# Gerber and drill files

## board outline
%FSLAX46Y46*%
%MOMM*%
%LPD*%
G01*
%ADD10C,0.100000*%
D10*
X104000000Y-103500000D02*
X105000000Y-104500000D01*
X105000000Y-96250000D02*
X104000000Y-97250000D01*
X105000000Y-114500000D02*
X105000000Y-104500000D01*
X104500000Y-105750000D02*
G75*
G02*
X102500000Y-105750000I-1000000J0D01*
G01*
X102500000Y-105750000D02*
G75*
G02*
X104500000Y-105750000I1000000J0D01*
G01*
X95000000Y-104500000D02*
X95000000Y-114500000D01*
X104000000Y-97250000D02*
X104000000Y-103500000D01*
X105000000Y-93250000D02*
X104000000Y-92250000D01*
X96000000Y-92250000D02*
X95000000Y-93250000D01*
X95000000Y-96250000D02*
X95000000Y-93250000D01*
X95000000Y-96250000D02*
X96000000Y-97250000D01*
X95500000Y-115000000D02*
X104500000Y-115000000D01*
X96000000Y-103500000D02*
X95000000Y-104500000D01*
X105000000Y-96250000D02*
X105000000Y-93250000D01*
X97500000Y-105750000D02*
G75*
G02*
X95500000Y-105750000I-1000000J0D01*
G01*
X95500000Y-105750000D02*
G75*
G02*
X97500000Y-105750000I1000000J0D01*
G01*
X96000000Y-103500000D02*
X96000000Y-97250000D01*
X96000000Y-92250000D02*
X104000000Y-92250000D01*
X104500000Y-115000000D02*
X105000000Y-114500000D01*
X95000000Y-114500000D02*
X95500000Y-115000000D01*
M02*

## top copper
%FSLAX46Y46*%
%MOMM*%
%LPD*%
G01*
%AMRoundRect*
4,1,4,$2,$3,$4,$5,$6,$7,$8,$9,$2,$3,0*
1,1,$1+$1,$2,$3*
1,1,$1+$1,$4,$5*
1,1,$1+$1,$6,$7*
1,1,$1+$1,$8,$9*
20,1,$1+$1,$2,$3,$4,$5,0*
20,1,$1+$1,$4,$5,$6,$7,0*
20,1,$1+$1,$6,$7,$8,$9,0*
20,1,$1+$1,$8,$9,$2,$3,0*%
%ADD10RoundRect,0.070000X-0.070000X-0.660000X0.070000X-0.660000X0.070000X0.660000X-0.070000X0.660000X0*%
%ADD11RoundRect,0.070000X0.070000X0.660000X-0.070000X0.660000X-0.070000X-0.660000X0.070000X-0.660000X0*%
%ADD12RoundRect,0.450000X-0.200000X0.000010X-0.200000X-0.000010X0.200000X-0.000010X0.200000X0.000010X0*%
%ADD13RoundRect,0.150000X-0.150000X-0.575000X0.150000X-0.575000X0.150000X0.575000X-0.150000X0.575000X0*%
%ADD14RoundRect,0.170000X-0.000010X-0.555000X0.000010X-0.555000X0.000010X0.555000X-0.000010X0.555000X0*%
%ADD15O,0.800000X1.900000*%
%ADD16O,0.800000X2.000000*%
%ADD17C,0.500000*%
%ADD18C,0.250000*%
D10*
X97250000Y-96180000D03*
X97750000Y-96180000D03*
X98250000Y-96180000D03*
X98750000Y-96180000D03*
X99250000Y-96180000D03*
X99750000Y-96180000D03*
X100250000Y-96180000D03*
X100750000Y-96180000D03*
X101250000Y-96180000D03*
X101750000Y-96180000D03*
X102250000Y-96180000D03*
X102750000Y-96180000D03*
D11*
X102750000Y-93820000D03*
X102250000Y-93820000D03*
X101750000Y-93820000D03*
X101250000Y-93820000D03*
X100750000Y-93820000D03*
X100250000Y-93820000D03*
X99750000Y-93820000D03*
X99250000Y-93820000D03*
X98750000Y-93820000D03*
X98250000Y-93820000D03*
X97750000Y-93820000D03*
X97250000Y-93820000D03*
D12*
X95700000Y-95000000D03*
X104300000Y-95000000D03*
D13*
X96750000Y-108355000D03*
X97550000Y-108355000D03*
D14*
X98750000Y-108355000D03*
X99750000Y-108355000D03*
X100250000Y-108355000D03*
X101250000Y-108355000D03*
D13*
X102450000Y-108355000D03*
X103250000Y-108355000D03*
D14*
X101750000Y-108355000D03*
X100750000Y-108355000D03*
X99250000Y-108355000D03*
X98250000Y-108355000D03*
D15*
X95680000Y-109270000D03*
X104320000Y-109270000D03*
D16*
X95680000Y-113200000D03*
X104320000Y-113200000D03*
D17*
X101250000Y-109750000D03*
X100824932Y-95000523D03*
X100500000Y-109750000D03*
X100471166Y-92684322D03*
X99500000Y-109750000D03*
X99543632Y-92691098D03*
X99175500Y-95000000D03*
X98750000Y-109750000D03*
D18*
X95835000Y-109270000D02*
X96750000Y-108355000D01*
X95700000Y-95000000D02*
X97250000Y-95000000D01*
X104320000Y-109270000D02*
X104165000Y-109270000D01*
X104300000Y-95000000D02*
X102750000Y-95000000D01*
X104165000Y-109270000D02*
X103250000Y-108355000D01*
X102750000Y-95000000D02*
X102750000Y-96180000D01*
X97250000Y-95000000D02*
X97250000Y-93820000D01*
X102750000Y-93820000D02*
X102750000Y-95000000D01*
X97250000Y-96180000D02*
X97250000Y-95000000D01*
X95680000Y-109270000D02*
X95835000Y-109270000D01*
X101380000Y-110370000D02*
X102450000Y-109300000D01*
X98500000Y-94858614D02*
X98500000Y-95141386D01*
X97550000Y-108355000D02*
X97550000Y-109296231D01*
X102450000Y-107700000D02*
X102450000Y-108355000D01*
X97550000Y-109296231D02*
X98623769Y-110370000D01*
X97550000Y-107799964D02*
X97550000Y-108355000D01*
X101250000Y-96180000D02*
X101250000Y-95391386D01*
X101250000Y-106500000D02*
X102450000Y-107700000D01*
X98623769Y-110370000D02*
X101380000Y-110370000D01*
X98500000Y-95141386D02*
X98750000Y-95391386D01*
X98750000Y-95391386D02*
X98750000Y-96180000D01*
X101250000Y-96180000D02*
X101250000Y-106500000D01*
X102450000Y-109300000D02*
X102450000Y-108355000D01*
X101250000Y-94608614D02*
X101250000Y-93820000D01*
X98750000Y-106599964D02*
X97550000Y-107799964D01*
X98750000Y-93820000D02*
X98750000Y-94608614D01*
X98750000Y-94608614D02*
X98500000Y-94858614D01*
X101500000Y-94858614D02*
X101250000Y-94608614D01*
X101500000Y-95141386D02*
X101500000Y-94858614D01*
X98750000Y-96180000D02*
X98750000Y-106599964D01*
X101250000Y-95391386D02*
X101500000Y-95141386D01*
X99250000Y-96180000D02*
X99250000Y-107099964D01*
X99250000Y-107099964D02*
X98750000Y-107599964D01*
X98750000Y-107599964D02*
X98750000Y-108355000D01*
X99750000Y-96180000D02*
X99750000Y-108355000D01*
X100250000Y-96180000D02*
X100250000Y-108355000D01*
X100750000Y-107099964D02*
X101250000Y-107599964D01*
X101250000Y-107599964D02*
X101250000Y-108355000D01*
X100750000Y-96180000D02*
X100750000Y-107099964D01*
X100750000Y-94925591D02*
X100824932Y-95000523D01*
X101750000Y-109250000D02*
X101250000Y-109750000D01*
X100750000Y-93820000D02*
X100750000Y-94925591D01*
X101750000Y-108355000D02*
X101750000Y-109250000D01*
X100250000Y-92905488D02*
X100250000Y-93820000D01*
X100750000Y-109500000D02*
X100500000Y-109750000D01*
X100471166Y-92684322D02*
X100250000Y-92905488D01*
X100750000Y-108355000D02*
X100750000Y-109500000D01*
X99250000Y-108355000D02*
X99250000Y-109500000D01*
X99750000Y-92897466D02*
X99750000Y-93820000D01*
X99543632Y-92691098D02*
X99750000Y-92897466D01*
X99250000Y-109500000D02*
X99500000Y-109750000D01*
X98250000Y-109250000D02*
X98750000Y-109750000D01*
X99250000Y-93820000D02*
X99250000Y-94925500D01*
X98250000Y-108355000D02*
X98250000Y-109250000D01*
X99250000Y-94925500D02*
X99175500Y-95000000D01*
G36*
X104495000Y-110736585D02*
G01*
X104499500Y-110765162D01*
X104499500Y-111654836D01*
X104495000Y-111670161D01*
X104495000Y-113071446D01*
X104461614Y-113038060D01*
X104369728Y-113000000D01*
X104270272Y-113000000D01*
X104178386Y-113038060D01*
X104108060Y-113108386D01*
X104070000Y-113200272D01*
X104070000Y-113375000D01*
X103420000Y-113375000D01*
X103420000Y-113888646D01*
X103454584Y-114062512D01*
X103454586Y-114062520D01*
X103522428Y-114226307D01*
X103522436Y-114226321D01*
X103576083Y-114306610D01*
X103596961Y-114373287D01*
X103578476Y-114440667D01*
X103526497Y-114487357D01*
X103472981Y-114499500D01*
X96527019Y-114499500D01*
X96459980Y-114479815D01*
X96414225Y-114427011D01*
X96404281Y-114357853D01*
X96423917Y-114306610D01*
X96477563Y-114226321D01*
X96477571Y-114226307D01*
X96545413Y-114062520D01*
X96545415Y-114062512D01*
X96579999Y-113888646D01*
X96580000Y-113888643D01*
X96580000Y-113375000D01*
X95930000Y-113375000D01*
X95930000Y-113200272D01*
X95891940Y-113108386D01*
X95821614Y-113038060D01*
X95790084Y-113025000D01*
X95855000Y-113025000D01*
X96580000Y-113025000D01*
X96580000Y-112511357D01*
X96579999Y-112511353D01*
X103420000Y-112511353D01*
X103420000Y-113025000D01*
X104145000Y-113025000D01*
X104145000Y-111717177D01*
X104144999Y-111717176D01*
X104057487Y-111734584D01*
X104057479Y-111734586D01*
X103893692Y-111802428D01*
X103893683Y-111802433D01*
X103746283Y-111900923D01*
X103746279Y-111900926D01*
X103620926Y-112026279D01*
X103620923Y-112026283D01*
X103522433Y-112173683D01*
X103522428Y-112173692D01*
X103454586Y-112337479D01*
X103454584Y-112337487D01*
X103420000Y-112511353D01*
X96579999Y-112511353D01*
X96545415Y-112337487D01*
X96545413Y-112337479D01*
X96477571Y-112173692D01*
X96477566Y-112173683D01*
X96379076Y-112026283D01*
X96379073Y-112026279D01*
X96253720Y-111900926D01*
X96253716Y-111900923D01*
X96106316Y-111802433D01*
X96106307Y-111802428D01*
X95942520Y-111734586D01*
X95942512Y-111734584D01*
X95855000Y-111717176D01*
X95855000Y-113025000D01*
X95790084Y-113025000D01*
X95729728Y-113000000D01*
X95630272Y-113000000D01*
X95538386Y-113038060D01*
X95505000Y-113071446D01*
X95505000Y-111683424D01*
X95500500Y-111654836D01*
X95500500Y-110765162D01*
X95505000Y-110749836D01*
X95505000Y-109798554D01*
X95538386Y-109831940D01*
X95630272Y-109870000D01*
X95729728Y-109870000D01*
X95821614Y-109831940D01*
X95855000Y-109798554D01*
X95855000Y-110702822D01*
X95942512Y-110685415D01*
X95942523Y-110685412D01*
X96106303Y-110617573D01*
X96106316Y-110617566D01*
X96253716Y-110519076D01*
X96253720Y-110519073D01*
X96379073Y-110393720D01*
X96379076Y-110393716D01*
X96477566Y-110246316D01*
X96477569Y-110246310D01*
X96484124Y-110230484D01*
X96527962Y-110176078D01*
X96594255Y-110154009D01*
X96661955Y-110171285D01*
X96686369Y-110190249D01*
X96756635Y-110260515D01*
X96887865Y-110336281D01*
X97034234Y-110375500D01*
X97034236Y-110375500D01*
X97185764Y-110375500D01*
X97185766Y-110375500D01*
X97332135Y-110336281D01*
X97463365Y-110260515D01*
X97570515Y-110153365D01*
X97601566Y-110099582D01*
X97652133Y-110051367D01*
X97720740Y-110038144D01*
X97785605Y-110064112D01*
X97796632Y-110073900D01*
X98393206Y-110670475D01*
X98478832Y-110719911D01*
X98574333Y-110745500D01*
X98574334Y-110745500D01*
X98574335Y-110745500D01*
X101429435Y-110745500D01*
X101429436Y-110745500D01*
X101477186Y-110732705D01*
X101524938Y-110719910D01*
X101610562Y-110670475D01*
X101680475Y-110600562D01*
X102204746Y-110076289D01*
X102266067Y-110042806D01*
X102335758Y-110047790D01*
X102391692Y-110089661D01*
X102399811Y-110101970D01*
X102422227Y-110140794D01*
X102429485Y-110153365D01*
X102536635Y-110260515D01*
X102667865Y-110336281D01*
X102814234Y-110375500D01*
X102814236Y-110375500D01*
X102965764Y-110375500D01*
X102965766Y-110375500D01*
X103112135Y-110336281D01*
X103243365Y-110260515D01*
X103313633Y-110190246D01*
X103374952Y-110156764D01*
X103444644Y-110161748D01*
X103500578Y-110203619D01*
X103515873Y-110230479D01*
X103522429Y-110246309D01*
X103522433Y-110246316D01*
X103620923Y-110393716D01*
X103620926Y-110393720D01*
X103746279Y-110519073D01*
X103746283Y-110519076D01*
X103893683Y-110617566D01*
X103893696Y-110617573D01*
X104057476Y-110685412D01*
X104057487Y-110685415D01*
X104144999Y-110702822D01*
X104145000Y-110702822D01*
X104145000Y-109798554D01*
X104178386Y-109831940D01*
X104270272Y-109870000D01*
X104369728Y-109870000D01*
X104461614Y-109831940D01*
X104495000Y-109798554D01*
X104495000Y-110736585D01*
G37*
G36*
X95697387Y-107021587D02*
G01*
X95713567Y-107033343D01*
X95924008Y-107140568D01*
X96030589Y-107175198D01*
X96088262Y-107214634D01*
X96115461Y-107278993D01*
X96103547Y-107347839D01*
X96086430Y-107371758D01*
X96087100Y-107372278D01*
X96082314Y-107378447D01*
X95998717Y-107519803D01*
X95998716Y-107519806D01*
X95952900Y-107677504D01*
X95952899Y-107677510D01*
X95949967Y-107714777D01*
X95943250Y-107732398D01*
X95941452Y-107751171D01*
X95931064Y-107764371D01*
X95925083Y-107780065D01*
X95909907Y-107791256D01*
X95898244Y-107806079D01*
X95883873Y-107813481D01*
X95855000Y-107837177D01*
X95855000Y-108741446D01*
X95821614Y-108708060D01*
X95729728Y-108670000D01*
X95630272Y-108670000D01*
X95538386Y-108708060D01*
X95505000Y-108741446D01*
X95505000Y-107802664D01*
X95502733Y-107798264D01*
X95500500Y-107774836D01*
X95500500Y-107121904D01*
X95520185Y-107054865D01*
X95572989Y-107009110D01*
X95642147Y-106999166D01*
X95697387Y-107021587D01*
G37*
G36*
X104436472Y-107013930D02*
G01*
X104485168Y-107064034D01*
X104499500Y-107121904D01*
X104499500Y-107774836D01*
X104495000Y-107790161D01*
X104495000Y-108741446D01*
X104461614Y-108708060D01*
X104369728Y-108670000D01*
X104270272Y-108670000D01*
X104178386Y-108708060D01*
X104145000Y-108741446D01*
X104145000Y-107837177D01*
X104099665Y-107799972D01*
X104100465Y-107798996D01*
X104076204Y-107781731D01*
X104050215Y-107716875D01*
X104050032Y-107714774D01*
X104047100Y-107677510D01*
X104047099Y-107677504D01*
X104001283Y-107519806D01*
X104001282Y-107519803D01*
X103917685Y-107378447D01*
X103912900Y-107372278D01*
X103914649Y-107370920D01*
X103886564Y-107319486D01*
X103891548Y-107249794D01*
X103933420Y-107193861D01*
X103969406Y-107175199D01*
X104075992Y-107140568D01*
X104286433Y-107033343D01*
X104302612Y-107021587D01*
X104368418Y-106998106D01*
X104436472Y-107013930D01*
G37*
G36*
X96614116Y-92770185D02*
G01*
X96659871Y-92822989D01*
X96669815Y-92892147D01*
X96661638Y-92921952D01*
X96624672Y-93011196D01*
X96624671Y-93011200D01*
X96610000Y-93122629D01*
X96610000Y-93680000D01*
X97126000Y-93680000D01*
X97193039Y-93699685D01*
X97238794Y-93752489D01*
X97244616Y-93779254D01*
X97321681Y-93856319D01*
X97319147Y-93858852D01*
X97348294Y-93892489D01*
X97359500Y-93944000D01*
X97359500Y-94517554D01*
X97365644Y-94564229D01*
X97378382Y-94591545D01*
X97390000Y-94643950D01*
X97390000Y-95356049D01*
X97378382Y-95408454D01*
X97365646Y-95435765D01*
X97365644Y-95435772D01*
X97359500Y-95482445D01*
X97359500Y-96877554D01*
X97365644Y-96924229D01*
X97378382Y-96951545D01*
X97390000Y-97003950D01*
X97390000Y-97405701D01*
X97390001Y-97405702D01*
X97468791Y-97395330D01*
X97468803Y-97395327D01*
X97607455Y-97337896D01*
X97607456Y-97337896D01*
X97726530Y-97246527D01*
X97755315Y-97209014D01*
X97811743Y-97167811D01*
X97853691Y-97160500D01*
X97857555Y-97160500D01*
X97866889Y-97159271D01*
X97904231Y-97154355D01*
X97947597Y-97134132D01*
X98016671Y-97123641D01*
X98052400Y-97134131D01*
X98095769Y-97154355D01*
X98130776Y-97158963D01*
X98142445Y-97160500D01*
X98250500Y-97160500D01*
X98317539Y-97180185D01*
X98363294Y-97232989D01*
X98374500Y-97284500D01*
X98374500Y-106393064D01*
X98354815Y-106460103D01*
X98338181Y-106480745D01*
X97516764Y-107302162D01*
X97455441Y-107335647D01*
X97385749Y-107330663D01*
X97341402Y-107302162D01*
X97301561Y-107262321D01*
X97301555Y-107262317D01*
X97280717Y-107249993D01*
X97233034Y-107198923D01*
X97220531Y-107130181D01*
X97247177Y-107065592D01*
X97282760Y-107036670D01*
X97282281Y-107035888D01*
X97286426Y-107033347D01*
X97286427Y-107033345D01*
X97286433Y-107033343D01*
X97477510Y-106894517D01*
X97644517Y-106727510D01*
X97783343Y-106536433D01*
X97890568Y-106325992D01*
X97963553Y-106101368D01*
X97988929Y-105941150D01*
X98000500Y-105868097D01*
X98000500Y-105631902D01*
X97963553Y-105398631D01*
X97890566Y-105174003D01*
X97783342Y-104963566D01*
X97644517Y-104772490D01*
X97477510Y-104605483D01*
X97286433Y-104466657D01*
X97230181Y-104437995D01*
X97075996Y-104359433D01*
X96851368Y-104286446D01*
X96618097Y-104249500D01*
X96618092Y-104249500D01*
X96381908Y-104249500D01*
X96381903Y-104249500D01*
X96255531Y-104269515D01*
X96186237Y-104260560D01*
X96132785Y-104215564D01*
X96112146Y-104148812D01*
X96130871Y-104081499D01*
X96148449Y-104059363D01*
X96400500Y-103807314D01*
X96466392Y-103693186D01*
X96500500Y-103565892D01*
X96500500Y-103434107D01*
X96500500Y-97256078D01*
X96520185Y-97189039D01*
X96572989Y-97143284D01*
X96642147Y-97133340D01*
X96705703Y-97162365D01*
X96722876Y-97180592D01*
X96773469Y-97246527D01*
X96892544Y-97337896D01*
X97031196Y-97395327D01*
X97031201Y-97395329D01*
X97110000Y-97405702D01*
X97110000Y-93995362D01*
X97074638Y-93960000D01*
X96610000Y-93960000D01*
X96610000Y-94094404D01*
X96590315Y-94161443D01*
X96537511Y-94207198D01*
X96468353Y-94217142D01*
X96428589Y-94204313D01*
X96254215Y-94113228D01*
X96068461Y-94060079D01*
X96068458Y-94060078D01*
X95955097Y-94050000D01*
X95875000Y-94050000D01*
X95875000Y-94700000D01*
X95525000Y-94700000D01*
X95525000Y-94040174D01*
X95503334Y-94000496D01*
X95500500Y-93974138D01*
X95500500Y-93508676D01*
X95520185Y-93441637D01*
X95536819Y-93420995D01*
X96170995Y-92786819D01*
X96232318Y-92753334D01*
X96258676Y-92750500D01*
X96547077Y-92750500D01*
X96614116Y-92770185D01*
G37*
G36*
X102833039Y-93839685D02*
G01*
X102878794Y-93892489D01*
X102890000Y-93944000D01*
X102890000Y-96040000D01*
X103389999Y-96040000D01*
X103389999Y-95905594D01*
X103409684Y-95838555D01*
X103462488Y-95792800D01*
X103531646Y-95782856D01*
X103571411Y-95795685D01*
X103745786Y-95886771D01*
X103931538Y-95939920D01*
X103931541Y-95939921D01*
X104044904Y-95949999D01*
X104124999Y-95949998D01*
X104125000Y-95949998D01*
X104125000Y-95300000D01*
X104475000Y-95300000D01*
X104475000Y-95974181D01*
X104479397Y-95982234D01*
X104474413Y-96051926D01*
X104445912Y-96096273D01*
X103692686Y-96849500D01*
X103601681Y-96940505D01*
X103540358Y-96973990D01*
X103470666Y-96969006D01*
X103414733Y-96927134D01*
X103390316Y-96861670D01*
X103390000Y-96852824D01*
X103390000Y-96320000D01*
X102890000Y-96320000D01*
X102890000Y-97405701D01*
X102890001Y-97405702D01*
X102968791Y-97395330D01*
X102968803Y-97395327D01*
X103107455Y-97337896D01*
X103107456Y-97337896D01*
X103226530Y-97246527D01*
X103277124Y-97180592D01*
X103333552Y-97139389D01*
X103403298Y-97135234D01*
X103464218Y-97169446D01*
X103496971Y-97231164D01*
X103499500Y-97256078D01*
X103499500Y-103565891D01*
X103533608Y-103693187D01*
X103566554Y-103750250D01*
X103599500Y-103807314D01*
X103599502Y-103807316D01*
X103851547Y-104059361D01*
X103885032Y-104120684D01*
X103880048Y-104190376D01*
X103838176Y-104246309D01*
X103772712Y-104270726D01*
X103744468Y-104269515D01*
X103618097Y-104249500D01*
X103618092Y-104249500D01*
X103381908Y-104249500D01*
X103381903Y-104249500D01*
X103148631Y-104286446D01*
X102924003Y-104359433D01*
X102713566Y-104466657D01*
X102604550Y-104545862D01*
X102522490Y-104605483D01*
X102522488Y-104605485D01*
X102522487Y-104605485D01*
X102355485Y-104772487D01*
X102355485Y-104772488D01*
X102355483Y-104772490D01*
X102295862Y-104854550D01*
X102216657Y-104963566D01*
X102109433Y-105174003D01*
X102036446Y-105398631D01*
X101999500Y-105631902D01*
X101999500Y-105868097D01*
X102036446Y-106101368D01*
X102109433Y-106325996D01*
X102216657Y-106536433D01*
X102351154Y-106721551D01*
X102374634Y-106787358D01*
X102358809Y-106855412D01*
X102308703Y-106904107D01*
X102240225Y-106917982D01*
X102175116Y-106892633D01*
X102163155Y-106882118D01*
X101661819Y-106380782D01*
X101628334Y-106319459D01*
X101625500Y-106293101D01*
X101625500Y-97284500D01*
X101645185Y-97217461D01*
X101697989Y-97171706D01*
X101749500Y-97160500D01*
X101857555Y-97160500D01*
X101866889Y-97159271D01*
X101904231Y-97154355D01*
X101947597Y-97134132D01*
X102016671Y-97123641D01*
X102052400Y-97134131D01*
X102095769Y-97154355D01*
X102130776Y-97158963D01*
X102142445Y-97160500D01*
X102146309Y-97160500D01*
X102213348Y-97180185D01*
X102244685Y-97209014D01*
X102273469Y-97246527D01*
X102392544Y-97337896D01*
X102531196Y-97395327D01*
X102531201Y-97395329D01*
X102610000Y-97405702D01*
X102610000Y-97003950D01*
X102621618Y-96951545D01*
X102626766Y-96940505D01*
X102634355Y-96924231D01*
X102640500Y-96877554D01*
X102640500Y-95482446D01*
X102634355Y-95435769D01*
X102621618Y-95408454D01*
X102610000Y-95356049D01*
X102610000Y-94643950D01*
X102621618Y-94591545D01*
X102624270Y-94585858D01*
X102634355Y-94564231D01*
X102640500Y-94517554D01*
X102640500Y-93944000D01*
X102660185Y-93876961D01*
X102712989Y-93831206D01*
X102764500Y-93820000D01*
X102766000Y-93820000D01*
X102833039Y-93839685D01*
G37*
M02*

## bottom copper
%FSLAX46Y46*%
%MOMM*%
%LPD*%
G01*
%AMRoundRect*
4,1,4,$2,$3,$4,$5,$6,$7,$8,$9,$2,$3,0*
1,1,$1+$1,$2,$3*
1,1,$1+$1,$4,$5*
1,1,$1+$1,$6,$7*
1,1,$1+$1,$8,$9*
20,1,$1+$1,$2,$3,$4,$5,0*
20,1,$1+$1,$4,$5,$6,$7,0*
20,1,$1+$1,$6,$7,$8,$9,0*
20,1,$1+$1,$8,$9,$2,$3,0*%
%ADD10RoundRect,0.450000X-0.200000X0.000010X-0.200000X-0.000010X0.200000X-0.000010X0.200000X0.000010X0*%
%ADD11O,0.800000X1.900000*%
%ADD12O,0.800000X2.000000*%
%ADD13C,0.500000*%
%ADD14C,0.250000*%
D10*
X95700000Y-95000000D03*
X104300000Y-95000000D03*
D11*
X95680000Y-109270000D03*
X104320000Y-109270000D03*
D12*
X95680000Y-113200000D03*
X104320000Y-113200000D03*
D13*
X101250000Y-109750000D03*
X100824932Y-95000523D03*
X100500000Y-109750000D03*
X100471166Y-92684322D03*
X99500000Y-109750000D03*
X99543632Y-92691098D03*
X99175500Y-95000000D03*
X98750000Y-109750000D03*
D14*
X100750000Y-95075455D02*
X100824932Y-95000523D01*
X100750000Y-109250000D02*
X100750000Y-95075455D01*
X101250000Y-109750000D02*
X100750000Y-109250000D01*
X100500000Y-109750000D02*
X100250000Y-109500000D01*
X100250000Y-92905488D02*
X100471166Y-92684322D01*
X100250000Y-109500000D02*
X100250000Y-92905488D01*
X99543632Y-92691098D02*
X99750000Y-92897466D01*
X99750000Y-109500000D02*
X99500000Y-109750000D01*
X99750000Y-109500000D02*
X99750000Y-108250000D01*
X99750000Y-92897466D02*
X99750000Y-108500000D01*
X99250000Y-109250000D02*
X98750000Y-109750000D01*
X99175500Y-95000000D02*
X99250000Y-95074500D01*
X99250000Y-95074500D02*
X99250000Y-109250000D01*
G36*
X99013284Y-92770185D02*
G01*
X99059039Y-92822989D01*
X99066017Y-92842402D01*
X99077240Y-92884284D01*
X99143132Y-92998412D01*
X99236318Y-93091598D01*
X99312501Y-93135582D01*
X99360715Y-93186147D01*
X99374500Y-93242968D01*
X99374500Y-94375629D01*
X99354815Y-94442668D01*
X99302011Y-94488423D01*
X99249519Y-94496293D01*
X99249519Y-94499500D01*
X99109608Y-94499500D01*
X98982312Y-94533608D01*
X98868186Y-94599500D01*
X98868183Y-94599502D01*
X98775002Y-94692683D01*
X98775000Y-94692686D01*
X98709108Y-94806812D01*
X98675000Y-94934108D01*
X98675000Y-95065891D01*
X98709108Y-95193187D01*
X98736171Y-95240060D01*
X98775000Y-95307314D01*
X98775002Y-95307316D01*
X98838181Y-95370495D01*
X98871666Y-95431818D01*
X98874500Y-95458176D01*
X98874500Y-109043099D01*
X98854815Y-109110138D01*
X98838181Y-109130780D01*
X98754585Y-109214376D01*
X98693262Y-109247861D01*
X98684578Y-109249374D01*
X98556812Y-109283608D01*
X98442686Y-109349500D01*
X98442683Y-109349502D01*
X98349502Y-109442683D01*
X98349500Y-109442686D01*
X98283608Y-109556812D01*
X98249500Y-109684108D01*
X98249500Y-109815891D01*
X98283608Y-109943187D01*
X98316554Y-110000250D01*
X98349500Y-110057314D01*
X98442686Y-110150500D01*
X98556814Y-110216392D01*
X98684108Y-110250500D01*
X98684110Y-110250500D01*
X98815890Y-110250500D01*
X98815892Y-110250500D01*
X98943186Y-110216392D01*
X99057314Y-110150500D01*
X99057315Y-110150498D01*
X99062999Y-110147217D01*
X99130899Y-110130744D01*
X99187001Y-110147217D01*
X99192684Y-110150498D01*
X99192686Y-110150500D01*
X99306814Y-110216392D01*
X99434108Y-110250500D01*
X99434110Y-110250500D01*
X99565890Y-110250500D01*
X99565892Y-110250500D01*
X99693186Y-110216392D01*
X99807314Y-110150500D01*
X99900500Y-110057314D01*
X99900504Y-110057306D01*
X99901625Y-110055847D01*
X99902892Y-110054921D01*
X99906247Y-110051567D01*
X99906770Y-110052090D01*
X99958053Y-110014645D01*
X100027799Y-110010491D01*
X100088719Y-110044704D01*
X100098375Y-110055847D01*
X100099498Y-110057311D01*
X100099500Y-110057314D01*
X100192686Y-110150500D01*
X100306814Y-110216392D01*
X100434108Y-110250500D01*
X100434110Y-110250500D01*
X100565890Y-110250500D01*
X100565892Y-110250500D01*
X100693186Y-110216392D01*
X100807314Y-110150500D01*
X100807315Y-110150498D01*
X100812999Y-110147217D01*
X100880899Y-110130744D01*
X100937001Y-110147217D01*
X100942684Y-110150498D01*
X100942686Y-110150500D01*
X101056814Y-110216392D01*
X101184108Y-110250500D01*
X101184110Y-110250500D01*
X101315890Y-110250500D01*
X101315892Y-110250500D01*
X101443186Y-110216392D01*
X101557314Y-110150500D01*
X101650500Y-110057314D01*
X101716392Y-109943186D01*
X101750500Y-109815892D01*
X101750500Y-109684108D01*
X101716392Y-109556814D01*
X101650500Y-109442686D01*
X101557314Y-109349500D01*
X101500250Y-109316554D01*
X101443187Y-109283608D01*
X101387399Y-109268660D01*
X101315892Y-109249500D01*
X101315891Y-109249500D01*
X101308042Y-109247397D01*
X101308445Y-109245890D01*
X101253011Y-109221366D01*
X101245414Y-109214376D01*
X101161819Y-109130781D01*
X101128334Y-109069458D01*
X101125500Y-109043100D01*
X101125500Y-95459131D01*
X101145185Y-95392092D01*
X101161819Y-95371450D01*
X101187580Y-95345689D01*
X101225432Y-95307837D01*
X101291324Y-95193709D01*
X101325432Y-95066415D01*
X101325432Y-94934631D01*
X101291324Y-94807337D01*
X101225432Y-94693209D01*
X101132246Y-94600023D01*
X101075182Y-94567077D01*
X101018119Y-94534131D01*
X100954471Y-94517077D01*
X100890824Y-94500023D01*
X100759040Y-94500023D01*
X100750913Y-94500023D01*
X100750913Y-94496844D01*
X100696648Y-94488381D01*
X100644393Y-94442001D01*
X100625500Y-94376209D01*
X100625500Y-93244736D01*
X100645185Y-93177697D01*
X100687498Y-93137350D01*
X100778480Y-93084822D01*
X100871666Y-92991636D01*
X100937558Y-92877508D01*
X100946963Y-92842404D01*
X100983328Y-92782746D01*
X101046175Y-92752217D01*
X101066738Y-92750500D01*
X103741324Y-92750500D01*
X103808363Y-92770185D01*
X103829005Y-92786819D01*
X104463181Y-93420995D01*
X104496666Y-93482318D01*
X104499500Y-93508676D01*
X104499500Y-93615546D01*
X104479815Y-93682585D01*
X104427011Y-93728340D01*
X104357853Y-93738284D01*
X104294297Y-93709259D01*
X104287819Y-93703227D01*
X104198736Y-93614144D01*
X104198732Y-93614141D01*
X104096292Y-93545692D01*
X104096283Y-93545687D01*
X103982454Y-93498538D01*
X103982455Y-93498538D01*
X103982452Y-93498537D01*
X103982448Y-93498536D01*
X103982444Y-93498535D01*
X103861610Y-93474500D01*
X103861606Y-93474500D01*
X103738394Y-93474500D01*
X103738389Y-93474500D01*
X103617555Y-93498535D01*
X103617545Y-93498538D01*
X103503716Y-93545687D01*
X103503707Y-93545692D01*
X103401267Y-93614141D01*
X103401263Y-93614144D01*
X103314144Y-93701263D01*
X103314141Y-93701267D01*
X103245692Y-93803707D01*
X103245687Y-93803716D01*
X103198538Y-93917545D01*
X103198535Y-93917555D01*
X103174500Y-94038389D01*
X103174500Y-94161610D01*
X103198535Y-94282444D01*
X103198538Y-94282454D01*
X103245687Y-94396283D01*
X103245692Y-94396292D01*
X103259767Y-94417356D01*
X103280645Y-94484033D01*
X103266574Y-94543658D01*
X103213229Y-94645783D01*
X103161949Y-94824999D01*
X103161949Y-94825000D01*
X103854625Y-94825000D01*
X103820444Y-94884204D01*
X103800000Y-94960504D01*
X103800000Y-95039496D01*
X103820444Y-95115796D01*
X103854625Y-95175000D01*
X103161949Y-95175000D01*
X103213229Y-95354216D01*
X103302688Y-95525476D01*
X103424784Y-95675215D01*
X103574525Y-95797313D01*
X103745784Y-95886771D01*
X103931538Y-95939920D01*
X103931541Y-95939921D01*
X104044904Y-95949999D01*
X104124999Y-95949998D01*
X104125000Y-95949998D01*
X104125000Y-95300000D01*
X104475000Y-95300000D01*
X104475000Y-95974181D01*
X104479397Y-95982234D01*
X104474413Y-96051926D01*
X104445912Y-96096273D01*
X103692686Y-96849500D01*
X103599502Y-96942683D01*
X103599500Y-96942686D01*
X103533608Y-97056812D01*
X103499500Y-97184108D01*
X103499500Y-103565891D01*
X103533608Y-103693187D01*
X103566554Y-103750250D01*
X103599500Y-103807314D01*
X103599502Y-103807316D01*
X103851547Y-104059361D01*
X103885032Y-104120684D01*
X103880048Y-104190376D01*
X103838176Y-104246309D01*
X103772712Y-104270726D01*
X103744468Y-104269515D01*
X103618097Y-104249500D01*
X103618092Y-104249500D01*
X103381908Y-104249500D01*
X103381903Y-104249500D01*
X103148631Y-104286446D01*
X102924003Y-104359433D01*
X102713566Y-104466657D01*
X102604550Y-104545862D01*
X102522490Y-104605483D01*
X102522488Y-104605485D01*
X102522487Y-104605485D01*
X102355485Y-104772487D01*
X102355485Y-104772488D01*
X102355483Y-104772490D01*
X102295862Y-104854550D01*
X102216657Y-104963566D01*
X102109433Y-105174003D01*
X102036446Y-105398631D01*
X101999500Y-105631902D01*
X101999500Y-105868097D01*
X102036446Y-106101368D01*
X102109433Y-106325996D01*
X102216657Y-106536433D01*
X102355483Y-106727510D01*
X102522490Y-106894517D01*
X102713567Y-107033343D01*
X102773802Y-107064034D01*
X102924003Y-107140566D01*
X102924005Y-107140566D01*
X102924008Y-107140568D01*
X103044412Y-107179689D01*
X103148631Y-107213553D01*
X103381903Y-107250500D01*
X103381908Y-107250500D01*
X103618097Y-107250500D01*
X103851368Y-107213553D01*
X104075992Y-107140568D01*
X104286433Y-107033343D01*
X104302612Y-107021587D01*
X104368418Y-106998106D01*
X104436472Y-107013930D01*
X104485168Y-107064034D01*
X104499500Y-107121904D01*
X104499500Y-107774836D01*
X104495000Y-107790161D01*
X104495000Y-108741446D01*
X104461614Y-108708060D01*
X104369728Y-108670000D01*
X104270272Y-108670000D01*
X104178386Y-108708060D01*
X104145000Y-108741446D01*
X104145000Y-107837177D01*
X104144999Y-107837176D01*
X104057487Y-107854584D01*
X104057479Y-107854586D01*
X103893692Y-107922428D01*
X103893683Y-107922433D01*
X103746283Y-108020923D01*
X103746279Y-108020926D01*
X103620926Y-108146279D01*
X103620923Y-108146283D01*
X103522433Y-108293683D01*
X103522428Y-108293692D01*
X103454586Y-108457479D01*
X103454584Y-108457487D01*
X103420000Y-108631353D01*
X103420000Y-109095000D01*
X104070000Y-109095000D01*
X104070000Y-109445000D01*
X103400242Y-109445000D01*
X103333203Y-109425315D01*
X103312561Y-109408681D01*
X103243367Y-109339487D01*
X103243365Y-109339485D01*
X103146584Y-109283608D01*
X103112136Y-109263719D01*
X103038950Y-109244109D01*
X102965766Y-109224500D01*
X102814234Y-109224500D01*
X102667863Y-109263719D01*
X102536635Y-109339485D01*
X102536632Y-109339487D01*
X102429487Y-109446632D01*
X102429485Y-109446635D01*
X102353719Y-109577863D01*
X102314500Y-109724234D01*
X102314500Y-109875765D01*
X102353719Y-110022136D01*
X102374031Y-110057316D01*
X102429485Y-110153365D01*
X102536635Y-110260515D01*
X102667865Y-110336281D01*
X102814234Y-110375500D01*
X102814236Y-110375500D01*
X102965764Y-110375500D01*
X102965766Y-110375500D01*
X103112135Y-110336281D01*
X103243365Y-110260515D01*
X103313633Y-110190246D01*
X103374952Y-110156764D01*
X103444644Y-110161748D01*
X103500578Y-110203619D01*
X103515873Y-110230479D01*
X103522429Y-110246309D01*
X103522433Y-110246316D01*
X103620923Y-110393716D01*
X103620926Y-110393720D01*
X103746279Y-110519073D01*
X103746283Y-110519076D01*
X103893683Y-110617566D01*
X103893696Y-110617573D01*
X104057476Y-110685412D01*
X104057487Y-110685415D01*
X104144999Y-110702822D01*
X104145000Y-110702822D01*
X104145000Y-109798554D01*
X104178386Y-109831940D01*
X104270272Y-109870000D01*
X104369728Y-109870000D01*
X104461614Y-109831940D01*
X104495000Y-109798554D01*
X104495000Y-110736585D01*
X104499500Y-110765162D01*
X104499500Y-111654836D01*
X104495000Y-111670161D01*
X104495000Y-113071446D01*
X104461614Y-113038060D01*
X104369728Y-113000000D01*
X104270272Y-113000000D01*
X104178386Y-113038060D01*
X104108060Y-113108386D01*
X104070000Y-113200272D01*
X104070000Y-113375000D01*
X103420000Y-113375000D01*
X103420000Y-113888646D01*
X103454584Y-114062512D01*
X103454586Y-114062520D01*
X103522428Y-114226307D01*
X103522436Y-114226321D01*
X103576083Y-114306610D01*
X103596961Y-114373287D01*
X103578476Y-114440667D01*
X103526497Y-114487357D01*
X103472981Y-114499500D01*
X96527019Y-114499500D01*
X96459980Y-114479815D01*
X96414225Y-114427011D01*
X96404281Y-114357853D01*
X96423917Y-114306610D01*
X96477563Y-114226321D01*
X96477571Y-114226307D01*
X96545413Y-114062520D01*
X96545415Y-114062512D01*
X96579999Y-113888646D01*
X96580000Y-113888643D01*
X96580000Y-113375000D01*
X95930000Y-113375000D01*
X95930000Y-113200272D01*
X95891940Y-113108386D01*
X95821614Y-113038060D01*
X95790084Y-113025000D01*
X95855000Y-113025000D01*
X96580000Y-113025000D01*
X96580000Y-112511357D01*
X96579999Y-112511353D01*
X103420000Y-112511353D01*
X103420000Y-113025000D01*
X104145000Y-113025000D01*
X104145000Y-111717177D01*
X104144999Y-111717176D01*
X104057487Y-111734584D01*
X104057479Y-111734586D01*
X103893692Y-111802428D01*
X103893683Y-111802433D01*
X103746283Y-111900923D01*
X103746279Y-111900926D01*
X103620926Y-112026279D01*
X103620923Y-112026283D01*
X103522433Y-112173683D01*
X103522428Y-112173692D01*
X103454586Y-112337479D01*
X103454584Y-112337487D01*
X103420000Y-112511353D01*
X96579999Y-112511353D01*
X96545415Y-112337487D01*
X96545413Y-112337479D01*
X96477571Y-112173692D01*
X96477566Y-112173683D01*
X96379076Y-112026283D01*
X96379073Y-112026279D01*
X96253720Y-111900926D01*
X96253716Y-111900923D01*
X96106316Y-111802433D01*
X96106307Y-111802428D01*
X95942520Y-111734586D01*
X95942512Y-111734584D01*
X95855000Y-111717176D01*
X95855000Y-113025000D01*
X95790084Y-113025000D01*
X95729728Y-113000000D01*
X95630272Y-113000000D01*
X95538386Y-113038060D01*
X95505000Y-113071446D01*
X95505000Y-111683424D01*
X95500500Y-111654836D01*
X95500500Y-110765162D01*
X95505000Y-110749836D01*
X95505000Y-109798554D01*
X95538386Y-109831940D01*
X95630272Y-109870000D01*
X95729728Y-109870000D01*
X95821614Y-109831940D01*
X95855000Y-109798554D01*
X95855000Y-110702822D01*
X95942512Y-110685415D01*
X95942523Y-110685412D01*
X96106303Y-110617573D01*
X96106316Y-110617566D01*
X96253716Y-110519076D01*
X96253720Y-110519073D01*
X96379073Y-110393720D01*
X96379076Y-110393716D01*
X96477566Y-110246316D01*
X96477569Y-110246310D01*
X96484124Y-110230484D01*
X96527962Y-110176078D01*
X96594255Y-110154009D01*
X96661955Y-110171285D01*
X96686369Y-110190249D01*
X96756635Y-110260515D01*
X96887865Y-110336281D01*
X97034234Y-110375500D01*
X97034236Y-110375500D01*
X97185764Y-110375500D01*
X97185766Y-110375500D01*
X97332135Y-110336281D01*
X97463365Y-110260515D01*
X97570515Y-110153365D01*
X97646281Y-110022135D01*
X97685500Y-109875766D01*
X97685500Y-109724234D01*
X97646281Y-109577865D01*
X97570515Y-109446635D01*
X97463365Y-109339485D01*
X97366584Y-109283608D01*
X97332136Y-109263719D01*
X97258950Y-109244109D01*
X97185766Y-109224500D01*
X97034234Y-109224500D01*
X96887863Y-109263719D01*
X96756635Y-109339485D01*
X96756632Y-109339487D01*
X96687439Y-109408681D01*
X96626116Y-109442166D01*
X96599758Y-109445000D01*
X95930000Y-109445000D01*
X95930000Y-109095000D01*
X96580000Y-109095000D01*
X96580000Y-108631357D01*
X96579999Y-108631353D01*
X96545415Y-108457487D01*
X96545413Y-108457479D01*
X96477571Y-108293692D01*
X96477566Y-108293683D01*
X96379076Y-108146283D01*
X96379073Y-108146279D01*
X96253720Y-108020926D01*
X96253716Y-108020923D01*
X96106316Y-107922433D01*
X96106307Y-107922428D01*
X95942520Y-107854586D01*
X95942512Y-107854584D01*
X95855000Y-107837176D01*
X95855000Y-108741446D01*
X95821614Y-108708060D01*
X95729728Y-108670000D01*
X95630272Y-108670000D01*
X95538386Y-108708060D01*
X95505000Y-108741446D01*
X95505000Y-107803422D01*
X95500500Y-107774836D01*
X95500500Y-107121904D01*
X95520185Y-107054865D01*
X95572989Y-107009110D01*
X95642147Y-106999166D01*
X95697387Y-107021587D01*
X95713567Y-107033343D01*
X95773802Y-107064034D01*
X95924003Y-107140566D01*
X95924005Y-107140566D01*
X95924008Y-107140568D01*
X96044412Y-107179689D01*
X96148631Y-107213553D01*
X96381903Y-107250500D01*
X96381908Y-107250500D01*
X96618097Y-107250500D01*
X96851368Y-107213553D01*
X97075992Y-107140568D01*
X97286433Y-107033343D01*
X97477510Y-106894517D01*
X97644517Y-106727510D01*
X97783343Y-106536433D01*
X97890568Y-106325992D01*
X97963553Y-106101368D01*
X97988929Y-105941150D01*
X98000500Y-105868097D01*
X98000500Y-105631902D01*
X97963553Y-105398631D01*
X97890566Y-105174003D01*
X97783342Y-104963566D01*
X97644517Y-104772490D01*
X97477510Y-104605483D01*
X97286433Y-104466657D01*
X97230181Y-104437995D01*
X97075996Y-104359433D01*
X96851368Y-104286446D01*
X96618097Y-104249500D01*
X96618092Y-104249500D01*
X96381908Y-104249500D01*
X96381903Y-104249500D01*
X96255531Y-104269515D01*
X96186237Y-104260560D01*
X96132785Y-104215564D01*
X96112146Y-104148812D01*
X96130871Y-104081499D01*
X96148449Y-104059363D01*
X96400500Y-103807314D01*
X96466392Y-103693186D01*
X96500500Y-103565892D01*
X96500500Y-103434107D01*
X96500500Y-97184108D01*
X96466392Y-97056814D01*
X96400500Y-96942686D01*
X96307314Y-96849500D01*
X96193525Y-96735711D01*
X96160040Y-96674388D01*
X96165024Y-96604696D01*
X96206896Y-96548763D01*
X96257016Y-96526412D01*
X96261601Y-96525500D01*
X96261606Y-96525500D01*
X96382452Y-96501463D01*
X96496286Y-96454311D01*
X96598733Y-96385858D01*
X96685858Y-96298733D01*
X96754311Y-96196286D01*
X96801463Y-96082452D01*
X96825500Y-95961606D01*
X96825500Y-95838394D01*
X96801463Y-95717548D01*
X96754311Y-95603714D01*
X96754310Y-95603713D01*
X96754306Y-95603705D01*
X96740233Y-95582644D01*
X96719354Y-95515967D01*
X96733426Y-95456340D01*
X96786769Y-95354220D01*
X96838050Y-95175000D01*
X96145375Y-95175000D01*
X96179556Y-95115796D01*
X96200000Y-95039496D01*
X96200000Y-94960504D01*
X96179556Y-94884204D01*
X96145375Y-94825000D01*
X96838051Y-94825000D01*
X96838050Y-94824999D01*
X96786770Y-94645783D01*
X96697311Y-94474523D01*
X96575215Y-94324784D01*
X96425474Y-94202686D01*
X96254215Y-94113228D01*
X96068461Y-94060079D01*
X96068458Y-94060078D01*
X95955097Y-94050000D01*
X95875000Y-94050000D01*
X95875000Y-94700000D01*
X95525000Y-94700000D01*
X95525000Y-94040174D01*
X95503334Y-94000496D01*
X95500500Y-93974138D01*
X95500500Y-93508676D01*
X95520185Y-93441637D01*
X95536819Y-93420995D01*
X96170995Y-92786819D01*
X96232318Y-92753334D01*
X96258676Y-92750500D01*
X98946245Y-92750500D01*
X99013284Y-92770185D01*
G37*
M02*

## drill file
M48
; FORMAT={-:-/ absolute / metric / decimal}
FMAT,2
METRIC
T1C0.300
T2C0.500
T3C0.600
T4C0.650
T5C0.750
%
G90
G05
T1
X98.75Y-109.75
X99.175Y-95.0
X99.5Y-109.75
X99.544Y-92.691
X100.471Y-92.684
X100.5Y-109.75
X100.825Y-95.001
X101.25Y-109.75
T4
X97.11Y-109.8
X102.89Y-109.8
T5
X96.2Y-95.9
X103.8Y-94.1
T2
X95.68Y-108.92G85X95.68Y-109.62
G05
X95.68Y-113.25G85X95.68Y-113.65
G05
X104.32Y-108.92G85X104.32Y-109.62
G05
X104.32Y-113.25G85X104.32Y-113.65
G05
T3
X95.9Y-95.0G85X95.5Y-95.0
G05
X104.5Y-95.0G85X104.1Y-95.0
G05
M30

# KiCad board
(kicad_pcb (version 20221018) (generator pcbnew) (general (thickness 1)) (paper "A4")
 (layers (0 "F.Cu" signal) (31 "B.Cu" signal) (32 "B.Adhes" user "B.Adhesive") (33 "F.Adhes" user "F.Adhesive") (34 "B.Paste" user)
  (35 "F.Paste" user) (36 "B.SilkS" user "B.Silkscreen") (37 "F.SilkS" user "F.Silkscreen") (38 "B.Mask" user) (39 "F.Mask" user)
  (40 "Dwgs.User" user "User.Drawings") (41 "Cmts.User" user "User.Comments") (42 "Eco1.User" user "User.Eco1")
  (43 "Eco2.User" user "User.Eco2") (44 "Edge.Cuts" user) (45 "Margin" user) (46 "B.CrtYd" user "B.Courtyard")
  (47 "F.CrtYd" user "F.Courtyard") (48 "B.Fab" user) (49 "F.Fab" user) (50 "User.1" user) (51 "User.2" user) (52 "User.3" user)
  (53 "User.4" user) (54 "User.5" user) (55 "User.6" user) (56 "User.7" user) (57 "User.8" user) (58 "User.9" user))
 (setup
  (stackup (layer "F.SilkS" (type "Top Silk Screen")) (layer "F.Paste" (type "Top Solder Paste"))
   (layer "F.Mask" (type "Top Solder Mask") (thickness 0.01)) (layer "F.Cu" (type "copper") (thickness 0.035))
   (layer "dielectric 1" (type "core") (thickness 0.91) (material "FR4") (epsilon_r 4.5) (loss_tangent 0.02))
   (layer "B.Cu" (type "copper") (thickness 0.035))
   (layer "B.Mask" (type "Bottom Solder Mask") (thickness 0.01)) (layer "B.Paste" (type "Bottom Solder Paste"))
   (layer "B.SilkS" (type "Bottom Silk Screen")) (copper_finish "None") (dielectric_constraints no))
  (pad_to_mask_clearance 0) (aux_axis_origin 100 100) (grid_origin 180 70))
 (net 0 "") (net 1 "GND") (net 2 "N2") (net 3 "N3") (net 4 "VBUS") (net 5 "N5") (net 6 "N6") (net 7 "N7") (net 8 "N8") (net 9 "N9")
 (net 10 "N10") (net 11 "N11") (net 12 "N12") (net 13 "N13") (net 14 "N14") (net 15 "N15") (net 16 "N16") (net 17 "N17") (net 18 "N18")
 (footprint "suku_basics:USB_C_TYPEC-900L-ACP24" (layer "F.Cu") (at 100 95 -90)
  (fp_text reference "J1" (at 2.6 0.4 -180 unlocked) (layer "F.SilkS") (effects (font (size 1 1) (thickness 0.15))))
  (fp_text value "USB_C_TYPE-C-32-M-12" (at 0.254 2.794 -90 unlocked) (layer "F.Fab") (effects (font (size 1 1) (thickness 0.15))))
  (pad "" np_thru_hole circle (at -0.9 -3.8 270) (size 0.75 0.75) (drill 0.75) (layers "F&B.Cu" "*.Mask"))
  (pad "" np_thru_hole circle (at 0.9 3.8 270) (size 0.75 0.75) (drill 0.75) (layers "F&B.Cu" "*.Mask"))
  (pad "A1" smd roundrect (at 1.18 2.75) (size 0.28 1.46) (layers "F.Cu" "F.Paste" "F.Mask") (roundrect_rratio 0.25) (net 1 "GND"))
  (pad "A2" smd roundrect (at 1.18 2.25) (size 0.28 1.46) (layers "F.Cu" "F.Paste" "F.Mask") (roundrect_rratio 0.25) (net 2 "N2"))
  (pad "A3" smd roundrect (at 1.18 1.75) (size 0.28 1.46) (layers "F.Cu" "F.Paste" "F.Mask") (roundrect_rratio 0.25) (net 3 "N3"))
  (pad "A4" smd roundrect (at 1.18 1.25) (size 0.28 1.46) (layers "F.Cu" "F.Paste" "F.Mask") (roundrect_rratio 0.25) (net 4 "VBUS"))
  (pad "A5" smd roundrect (at 1.18 0.75) (size 0.28 1.46) (layers "F.Cu" "F.Paste" "F.Mask") (roundrect_rratio 0.25) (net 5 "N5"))
  (pad "A6" smd roundrect (at 1.18 0.25) (size 0.28 1.46) (layers "F.Cu" "F.Paste" "F.Mask") (roundrect_rratio 0.25) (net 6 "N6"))
  (pad "A7" smd roundrect (at 1.18 -0.25) (size 0.28 1.46) (layers "F.Cu" "F.Paste" "F.Mask") (roundrect_rratio 0.25) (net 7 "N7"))
  (pad "A8" smd roundrect (at 1.18 -0.75) (size 0.28 1.46) (layers "F.Cu" "F.Paste" "F.Mask") (roundrect_rratio 0.25) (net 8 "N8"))
  (pad "A9" smd roundrect (at 1.18 -1.25) (size 0.28 1.46) (layers "F.Cu" "F.Paste" "F.Mask") (roundrect_rratio 0.25) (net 4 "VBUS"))
  (pad "A10" smd roundrect (at 1.18 -1.75) (size 0.28 1.46) (layers "F.Cu" "F.Paste" "F.Mask") (roundrect_rratio 0.25) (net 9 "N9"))
  (pad "A11" smd roundrect (at 1.18 -2.25) (size 0.28 1.46) (layers "F.Cu" "F.Paste" "F.Mask") (roundrect_rratio 0.25) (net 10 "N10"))
  (pad "A12" smd roundrect (at 1.18 -2.75) (size 0.28 1.46) (layers "F.Cu" "F.Paste" "F.Mask") (roundrect_rratio 0.25) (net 1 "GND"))
  (pad "B1" smd roundrect (at -1.18 -2.75 180) (size 0.28 1.46) (layers "F.Cu" "F.Paste" "F.Mask") (roundrect_rratio 0.25) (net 1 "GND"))
  (pad "B2" smd roundrect (at -1.18 -2.25 180) (size 0.28 1.46) (layers "F.Cu" "F.Paste" "F.Mask") (roundrect_rratio 0.25) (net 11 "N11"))
  (pad "B3" smd roundrect (at -1.18 -1.75 180) (size 0.28 1.46) (layers "F.Cu" "F.Paste" "F.Mask") (roundrect_rratio 0.25) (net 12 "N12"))
  (pad "B4" smd roundrect (at -1.18 -1.25 180) (size 0.28 1.46) (layers "F.Cu" "F.Paste" "F.Mask") (roundrect_rratio 0.25) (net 4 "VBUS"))
  (pad "B5" smd roundrect (at -1.18 -0.75 180) (size 0.28 1.46) (layers "F.Cu" "F.Paste" "F.Mask") (roundrect_rratio 0.25) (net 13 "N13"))
  (pad "B6" smd roundrect (at -1.18 -0.25 180) (size 0.28 1.46) (layers "F.Cu" "F.Paste" "F.Mask") (roundrect_rratio 0.25) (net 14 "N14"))
  (pad "B7" smd roundrect (at -1.18 0.25 180) (size 0.28 1.46) (layers "F.Cu" "F.Paste" "F.Mask") (roundrect_rratio 0.25) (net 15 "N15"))
  (pad "B8" smd roundrect (at -1.18 0.75 180) (size 0.28 1.46) (layers "F.Cu" "F.Paste" "F.Mask") (roundrect_rratio 0.25) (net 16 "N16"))
  (pad "B9" smd roundrect (at -1.18 1.25 180) (size 0.28 1.46) (layers "F.Cu" "F.Paste" "F.Mask") (roundrect_rratio 0.25) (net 4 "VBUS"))
  (pad "B10" smd roundrect (at -1.18 1.75 180) (size 0.28 1.46) (layers "F.Cu" "F.Paste" "F.Mask") (roundrect_rratio 0.25) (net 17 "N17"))
  (pad "B11" smd roundrect (at -1.18 2.25 180) (size 0.28 1.46) (layers "F.Cu" "F.Paste" "F.Mask") (roundrect_rratio 0.25) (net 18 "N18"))
  (pad "B12" smd roundrect (at -1.18 2.75 180) (size 0.28 1.46) (layers "F.Cu" "F.Paste" "F.Mask") (roundrect_rratio 0.25) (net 1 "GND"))
  (pad "S1" thru_hole roundrect (at 0 4.3 270) (size 0.9 1.3) (drill oval 0.6 1) (layers "*.Cu" "*.Mask") (roundrect_rratio 0.5)
   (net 1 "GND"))
  (pad "S2" thru_hole roundrect (at 0 -4.3 270) (size 0.9 1.3) (drill oval 0.6 1) (layers "*.Cu" "*.Mask") (roundrect_rratio 0.5)
   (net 1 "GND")))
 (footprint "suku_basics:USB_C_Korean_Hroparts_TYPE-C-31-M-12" (layer "F.Cu") (at 100 111.25)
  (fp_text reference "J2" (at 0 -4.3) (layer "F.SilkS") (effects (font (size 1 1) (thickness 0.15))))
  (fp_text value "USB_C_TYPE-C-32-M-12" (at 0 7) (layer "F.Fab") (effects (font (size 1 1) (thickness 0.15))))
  (pad "" np_thru_hole circle (at -2.89 -1.45) (size 0.65 0.65) (drill 0.65) (layers "*.Cu" "*.Mask"))
  (pad "" np_thru_hole circle (at 2.89 -1.45) (size 0.65 0.65) (drill 0.65) (layers "*.Cu" "*.Mask"))
  (pad "A1B12" smd roundrect (at -3.25 -2.895) (size 0.6 1.45) (layers "F.Cu" "F.Paste" "F.Mask") (roundrect_rratio 0.25) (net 1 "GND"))
  (pad "A4B9" smd roundrect (at -2.45 -2.895) (size 0.6 1.45) (layers "F.Cu" "F.Paste" "F.Mask") (roundrect_rratio 0.25) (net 4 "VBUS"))
  (pad "A5" smd roundrect (at -1.25 -2.895) (size 0.34 1.45) (layers "F.Cu" "F.Paste" "F.Mask") (roundrect_rratio 0.5) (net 5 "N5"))
  (pad "A6" smd roundrect (at -0.25 -2.895) (size 0.34 1.45) (layers "F.Cu" "F.Paste" "F.Mask") (roundrect_rratio 0.5) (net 6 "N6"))
  (pad "A7" smd roundrect (at 0.25 -2.895) (size 0.34 1.45) (layers "F.Cu" "F.Paste" "F.Mask") (roundrect_rratio 0.5) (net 7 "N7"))
  (pad "A8" smd roundrect (at 1.25 -2.895) (size 0.34 1.45) (layers "F.Cu" "F.Paste" "F.Mask") (roundrect_rratio 0.5) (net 8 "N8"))
  (pad "A9B4" smd roundrect (at 2.45 -2.895) (size 0.6 1.45) (layers "F.Cu" "F.Paste" "F.Mask") (roundrect_rratio 0.25) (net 4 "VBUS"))
  (pad "A12B1" smd roundrect (at 3.25 -2.895) (size 0.6 1.45) (layers "F.Cu" "F.Paste" "F.Mask") (roundrect_rratio 0.25) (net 1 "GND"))
  (pad "B5" smd roundrect (at 1.75 -2.895) (size 0.34 1.45) (layers "F.Cu" "F.Paste" "F.Mask") (roundrect_rratio 0.5) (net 13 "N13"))
  (pad "B6" smd roundrect (at 0.75 -2.895) (size 0.34 1.45) (layers "F.Cu" "F.Paste" "F.Mask") (roundrect_rratio 0.5) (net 14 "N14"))
  (pad "B7" smd roundrect (at -0.75 -2.895) (size 0.34 1.45) (layers "F.Cu" "F.Paste" "F.Mask") (roundrect_rratio 0.5) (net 15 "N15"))
  (pad "B8" smd roundrect (at -1.75 -2.895) (size 0.34 1.45) (layers "F.Cu" "F.Paste" "F.Mask") (roundrect_rratio 0.5) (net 16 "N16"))
  (pad "S1" thru_hole oval (at -4.32 -1.98) (size 0.8 1.9) (drill oval 0.5 1.2) (layers "*.Cu" "*.Mask" "F.Paste") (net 1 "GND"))
  (pad "S2" thru_hole oval (at 4.32 -1.98) (size 0.8 1.9) (drill oval 0.5 1.2) (layers "*.Cu" "*.Mask" "F.Paste") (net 1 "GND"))
  (pad "S3" thru_hole oval (at -4.32 2.2) (size 0.8 2) (drill oval 0.5 0.9 (offset 0 -0.25)) (layers "*.Cu" "*.Mask" "F.Paste")
   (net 1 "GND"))
  (pad "S4" thru_hole oval (at 4.32 2.2) (size 0.8 2) (drill oval 0.5 0.9 (offset 0 -0.25)) (layers "*.Cu" "*.Mask" "F.Paste") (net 1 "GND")))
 (gr_line (start 104 103.5) (end 105 104.5) (stroke (width 0.1) (type default)) (layer "Edge.Cuts"))
 (gr_line (start 105 96.25) (end 104 97.25) (stroke (width 0.1) (type default)) (layer "Edge.Cuts"))
 (gr_line (start 105 114.5) (end 105 104.5) (stroke (width 0.1) (type default)) (layer "Edge.Cuts"))
 (gr_circle (center 103.5 105.75) (end 104.5 105.75) (stroke (width 0.1) (type default)) (fill none) (layer "Edge.Cuts"))
 (gr_line (start 95 104.5) (end 95 114.5) (stroke (width 0.1) (type default)) (layer "Edge.Cuts"))
 (gr_line (start 104 97.25) (end 104 103.5) (stroke (width 0.1) (type default)) (layer "Edge.Cuts"))
 (gr_line (start 105 93.25) (end 104 92.25) (stroke (width 0.1) (type default)) (layer "Edge.Cuts"))
 (gr_line (start 96 92.25) (end 95 93.25) (stroke (width 0.1) (type default)) (layer "Edge.Cuts"))
 (gr_line (start 95 96.25) (end 95 93.25) (stroke (width 0.1) (type default)) (layer "Edge.Cuts"))
 (gr_line (start 95 96.25) (end 96 97.25) (stroke (width 0.1) (type default)) (layer "Edge.Cuts"))
 (gr_line (start 95.5 115) (end 104.5 115) (stroke (width 0.1) (type default)) (layer "Edge.Cuts"))
 (gr_line (start 96 103.5) (end 95 104.5) (stroke (width 0.1) (type default)) (layer "Edge.Cuts"))
 (gr_line (start 105 96.25) (end 105 93.25) (stroke (width 0.1) (type default)) (layer "Edge.Cuts"))
 (gr_circle (center 96.5 105.75) (end 97.5 105.75) (stroke (width 0.1) (type default)) (fill none) (layer "Edge.Cuts"))
 (gr_line (start 96 103.5) (end 96 97.25) (stroke (width 0.1) (type default)) (layer "Edge.Cuts"))
 (gr_line (start 96 92.25) (end 104 92.25) (stroke (width 0.1) (type default)) (layer "Edge.Cuts"))
 (gr_line (start 104.5 115) (end 105 114.5) (stroke (width 0.1) (type default)) (layer "Edge.Cuts"))
 (gr_line (start 95 114.5) (end 95.5 115) (stroke (width 0.1) (type default)) (layer "Edge.Cuts"))
 (segment (start 95.835 109.27) (end 96.75 108.355) (width 0.25) (layer "F.Cu") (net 1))
 (segment (start 95.7 95) (end 97.25 95) (width 0.25) (layer "F.Cu") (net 1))
 (segment (start 104.32 109.27) (end 104.165 109.27) (width 0.25) (layer "F.Cu") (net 1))
 (segment (start 104.3 95) (end 102.75 95) (width 0.25) (layer "F.Cu") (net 1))
 (segment (start 104.165 109.27) (end 103.25 108.355) (width 0.25) (layer "F.Cu") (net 1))
 (segment (start 102.75 95) (end 102.75 96.18) (width 0.25) (layer "F.Cu") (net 1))
 (segment (start 97.25 95) (end 97.25 93.82) (width 0.25) (layer "F.Cu") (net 1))
 (segment (start 102.75 93.82) (end 102.75 95) (width 0.25) (layer "F.Cu") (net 1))
 (segment (start 97.25 96.18) (end 97.25 95) (width 0.25) (layer "F.Cu") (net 1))
 (segment (start 95.68 109.27) (end 95.835 109.27) (width 0.25) (layer "F.Cu") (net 1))
 (segment (start 101.38 110.37) (end 102.45 109.3) (width 0.25) (layer "F.Cu") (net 4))
 (segment (start 98.5 94.858614) (end 98.5 95.141386) (width 0.25) (layer "F.Cu") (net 4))
 (segment (start 97.55 108.355) (end 97.55 109.296231) (width 0.25) (layer "F.Cu") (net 4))
 (segment (start 102.45 107.7) (end 102.45 108.355) (width 0.25) (layer "F.Cu") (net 4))
 (segment (start 97.55 109.296231) (end 98.623769 110.37) (width 0.25) (layer "F.Cu") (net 4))
 (segment (start 97.55 107.799964) (end 97.55 108.355) (width 0.25) (layer "F.Cu") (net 4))
 (segment (start 101.25 96.18) (end 101.25 95.391386) (width 0.25) (layer "F.Cu") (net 4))
 (segment (start 101.25 106.5) (end 102.45 107.7) (width 0.25) (layer "F.Cu") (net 4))
 (segment (start 98.623769 110.37) (end 101.38 110.37) (width 0.25) (layer "F.Cu") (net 4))
 (segment (start 98.5 95.141386) (end 98.75 95.391386) (width 0.25) (layer "F.Cu") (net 4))
 (segment (start 98.75 95.391386) (end 98.75 96.18) (width 0.25) (layer "F.Cu") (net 4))
 (segment (start 101.25 96.18) (end 101.25 106.5) (width 0.25) (layer "F.Cu") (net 4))
 (segment (start 102.45 109.3) (end 102.45 108.355) (width 0.25) (layer "F.Cu") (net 4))
 (segment (start 101.25 94.608614) (end 101.25 93.82) (width 0.25) (layer "F.Cu") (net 4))
 (segment (start 98.75 106.599964) (end 97.55 107.799964) (width 0.25) (layer "F.Cu") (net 4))
 (segment (start 98.75 93.82) (end 98.75 94.608614) (width 0.25) (layer "F.Cu") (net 4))
 (segment (start 98.75 94.608614) (end 98.5 94.858614) (width 0.25) (layer "F.Cu") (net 4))
 (segment (start 101.5 94.858614) (end 101.25 94.608614) (width 0.25) (layer "F.Cu") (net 4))
 (segment (start 101.5 95.141386) (end 101.5 94.858614) (width 0.25) (layer "F.Cu") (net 4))
 (segment (start 98.75 96.18) (end 98.75 106.599964) (width 0.25) (layer "F.Cu") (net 4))
 (segment (start 101.25 95.391386) (end 101.5 95.141386) (width 0.25) (layer "F.Cu") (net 4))
 (segment (start 99.25 96.18) (end 99.25 107.099964) (width 0.25) (layer "F.Cu") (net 5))
 (segment (start 99.25 107.099964) (end 98.75 107.599964) (width 0.25) (layer "F.Cu") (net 5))
 (segment (start 98.75 107.599964) (end 98.75 108.355) (width 0.25) (layer "F.Cu") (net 5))
 (segment (start 99.75 96.18) (end 99.75 108.355) (width 0.25) (layer "F.Cu") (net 6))
 (segment (start 100.25 96.18) (end 100.25 108.355) (width 0.25) (layer "F.Cu") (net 7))
 (segment (start 100.75 107.099964) (end 101.25 107.599964) (width 0.25) (layer "F.Cu") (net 8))
 (segment (start 101.25 107.599964) (end 101.25 108.355) (width 0.25) (layer "F.Cu") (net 8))
 (segment (start 100.75 96.18) (end 100.75 107.099964) (width 0.25) (layer "F.Cu") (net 8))
 (segment (start 100.75 94.925591) (end 100.824932 95.000523) (width 0.25) (layer "F.Cu") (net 13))
 (segment (start 101.75 109.25) (end 101.25 109.75) (width 0.25) (layer "F.Cu") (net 13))
 (segment (start 100.75 93.82) (end 100.75 94.925591) (width 0.25) (layer "F.Cu") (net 13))
 (segment (start 101.75 108.355) (end 101.75 109.25) (width 0.25) (layer "F.Cu") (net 13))
 (via (at 101.25 109.75) (size 0.5) (drill 0.3) (layers "F.Cu" "B.Cu") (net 13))
 (via (at 100.824932 95.000523) (size 0.5) (drill 0.3) (layers "F.Cu" "B.Cu") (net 13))
 (segment (start 100.75 95.075455) (end 100.824932 95.000523) (width 0.25) (layer "B.Cu") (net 13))
 (segment (start 100.75 109.25) (end 100.75 95.075455) (width 0.25) (layer "B.Cu") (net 13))
 (segment (start 101.25 109.75) (end 100.75 109.25) (width 0.25) (layer "B.Cu") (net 13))
 (segment (start 100.25 92.905488) (end 100.25 93.82) (width 0.25) (layer "F.Cu") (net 14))
 (segment (start 100.75 109.5) (end 100.5 109.75) (width 0.25) (layer "F.Cu") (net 14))
 (segment (start 100.471166 92.684322) (end 100.25 92.905488) (width 0.25) (layer "F.Cu") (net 14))
 (segment (start 100.75 108.355) (end 100.75 109.5) (width 0.25) (layer "F.Cu") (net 14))
 (via (at 100.5 109.75) (size 0.5) (drill 0.3) (layers "F.Cu" "B.Cu") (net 14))
 (via (at 100.471166 92.684322) (size 0.5) (drill 0.3) (layers "F.Cu" "B.Cu") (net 14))
 (segment (start 100.5 109.75) (end 100.25 109.5) (width 0.25) (layer "B.Cu") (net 14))
 (segment (start 100.25 92.905488) (end 100.471166 92.684322) (width 0.25) (layer "B.Cu") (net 14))
 (segment (start 100.25 109.5) (end 100.25 92.905488) (width 0.25) (layer "B.Cu") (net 14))
 (segment (start 99.25 108.355) (end 99.25 109.5) (width 0.25) (layer "F.Cu") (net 15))
 (segment (start 99.75 92.897466) (end 99.75 93.82) (width 0.25) (layer "F.Cu") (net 15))
 (segment (start 99.543632 92.691098) (end 99.75 92.897466) (width 0.25) (layer "F.Cu") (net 15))
 (segment (start 99.25 109.5) (end 99.5 109.75) (width 0.25) (layer "F.Cu") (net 15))
 (via (at 99.5 109.75) (size 0.5) (drill 0.3) (layers "F.Cu" "B.Cu") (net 15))
 (via (at 99.543632 92.691098) (size 0.5) (drill 0.3) (layers "F.Cu" "B.Cu") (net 15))
 (segment (start 99.543632 92.691098) (end 99.75 92.897466) (width 0.25) (layer "B.Cu") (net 15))
 (segment (start 99.75 109.5) (end 99.5 109.75) (width 0.25) (layer "B.Cu") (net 15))
 (segment (start 99.75 109.5) (end 99.75 108.25) (width 0.25) (layer "B.Cu") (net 15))
 (segment (start 99.75 92.897466) (end 99.75 108.5) (width 0.25) (layer "B.Cu") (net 15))
 (segment (start 98.25 109.25) (end 98.75 109.75) (width 0.25) (layer "F.Cu") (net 16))
 (segment (start 99.25 93.82) (end 99.25 94.9255) (width 0.25) (layer "F.Cu") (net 16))
 (segment (start 98.25 108.355) (end 98.25 109.25) (width 0.25) (layer "F.Cu") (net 16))
 (segment (start 99.25 94.9255) (end 99.1755 95) (width 0.25) (layer "F.Cu") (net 16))
 (via (at 99.1755 95) (size 0.5) (drill 0.3) (layers "F.Cu" "B.Cu") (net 16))
 (via (at 98.75 109.75) (size 0.5) (drill 0.3) (layers "F.Cu" "B.Cu") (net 16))
 (segment (start 99.25 109.25) (end 98.75 109.75) (width 0.25) (layer "B.Cu") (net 16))
 (segment (start 99.1755 95) (end 99.25 95.0745) (width 0.25) (layer "B.Cu") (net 16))
 (segment (start 99.25 95.0745) (end 99.25 109.25) (width 0.25) (layer "B.Cu") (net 16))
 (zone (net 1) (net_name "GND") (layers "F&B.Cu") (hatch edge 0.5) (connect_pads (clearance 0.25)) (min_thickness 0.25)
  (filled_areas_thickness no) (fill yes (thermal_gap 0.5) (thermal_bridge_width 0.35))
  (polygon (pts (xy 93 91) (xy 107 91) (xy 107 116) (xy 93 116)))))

